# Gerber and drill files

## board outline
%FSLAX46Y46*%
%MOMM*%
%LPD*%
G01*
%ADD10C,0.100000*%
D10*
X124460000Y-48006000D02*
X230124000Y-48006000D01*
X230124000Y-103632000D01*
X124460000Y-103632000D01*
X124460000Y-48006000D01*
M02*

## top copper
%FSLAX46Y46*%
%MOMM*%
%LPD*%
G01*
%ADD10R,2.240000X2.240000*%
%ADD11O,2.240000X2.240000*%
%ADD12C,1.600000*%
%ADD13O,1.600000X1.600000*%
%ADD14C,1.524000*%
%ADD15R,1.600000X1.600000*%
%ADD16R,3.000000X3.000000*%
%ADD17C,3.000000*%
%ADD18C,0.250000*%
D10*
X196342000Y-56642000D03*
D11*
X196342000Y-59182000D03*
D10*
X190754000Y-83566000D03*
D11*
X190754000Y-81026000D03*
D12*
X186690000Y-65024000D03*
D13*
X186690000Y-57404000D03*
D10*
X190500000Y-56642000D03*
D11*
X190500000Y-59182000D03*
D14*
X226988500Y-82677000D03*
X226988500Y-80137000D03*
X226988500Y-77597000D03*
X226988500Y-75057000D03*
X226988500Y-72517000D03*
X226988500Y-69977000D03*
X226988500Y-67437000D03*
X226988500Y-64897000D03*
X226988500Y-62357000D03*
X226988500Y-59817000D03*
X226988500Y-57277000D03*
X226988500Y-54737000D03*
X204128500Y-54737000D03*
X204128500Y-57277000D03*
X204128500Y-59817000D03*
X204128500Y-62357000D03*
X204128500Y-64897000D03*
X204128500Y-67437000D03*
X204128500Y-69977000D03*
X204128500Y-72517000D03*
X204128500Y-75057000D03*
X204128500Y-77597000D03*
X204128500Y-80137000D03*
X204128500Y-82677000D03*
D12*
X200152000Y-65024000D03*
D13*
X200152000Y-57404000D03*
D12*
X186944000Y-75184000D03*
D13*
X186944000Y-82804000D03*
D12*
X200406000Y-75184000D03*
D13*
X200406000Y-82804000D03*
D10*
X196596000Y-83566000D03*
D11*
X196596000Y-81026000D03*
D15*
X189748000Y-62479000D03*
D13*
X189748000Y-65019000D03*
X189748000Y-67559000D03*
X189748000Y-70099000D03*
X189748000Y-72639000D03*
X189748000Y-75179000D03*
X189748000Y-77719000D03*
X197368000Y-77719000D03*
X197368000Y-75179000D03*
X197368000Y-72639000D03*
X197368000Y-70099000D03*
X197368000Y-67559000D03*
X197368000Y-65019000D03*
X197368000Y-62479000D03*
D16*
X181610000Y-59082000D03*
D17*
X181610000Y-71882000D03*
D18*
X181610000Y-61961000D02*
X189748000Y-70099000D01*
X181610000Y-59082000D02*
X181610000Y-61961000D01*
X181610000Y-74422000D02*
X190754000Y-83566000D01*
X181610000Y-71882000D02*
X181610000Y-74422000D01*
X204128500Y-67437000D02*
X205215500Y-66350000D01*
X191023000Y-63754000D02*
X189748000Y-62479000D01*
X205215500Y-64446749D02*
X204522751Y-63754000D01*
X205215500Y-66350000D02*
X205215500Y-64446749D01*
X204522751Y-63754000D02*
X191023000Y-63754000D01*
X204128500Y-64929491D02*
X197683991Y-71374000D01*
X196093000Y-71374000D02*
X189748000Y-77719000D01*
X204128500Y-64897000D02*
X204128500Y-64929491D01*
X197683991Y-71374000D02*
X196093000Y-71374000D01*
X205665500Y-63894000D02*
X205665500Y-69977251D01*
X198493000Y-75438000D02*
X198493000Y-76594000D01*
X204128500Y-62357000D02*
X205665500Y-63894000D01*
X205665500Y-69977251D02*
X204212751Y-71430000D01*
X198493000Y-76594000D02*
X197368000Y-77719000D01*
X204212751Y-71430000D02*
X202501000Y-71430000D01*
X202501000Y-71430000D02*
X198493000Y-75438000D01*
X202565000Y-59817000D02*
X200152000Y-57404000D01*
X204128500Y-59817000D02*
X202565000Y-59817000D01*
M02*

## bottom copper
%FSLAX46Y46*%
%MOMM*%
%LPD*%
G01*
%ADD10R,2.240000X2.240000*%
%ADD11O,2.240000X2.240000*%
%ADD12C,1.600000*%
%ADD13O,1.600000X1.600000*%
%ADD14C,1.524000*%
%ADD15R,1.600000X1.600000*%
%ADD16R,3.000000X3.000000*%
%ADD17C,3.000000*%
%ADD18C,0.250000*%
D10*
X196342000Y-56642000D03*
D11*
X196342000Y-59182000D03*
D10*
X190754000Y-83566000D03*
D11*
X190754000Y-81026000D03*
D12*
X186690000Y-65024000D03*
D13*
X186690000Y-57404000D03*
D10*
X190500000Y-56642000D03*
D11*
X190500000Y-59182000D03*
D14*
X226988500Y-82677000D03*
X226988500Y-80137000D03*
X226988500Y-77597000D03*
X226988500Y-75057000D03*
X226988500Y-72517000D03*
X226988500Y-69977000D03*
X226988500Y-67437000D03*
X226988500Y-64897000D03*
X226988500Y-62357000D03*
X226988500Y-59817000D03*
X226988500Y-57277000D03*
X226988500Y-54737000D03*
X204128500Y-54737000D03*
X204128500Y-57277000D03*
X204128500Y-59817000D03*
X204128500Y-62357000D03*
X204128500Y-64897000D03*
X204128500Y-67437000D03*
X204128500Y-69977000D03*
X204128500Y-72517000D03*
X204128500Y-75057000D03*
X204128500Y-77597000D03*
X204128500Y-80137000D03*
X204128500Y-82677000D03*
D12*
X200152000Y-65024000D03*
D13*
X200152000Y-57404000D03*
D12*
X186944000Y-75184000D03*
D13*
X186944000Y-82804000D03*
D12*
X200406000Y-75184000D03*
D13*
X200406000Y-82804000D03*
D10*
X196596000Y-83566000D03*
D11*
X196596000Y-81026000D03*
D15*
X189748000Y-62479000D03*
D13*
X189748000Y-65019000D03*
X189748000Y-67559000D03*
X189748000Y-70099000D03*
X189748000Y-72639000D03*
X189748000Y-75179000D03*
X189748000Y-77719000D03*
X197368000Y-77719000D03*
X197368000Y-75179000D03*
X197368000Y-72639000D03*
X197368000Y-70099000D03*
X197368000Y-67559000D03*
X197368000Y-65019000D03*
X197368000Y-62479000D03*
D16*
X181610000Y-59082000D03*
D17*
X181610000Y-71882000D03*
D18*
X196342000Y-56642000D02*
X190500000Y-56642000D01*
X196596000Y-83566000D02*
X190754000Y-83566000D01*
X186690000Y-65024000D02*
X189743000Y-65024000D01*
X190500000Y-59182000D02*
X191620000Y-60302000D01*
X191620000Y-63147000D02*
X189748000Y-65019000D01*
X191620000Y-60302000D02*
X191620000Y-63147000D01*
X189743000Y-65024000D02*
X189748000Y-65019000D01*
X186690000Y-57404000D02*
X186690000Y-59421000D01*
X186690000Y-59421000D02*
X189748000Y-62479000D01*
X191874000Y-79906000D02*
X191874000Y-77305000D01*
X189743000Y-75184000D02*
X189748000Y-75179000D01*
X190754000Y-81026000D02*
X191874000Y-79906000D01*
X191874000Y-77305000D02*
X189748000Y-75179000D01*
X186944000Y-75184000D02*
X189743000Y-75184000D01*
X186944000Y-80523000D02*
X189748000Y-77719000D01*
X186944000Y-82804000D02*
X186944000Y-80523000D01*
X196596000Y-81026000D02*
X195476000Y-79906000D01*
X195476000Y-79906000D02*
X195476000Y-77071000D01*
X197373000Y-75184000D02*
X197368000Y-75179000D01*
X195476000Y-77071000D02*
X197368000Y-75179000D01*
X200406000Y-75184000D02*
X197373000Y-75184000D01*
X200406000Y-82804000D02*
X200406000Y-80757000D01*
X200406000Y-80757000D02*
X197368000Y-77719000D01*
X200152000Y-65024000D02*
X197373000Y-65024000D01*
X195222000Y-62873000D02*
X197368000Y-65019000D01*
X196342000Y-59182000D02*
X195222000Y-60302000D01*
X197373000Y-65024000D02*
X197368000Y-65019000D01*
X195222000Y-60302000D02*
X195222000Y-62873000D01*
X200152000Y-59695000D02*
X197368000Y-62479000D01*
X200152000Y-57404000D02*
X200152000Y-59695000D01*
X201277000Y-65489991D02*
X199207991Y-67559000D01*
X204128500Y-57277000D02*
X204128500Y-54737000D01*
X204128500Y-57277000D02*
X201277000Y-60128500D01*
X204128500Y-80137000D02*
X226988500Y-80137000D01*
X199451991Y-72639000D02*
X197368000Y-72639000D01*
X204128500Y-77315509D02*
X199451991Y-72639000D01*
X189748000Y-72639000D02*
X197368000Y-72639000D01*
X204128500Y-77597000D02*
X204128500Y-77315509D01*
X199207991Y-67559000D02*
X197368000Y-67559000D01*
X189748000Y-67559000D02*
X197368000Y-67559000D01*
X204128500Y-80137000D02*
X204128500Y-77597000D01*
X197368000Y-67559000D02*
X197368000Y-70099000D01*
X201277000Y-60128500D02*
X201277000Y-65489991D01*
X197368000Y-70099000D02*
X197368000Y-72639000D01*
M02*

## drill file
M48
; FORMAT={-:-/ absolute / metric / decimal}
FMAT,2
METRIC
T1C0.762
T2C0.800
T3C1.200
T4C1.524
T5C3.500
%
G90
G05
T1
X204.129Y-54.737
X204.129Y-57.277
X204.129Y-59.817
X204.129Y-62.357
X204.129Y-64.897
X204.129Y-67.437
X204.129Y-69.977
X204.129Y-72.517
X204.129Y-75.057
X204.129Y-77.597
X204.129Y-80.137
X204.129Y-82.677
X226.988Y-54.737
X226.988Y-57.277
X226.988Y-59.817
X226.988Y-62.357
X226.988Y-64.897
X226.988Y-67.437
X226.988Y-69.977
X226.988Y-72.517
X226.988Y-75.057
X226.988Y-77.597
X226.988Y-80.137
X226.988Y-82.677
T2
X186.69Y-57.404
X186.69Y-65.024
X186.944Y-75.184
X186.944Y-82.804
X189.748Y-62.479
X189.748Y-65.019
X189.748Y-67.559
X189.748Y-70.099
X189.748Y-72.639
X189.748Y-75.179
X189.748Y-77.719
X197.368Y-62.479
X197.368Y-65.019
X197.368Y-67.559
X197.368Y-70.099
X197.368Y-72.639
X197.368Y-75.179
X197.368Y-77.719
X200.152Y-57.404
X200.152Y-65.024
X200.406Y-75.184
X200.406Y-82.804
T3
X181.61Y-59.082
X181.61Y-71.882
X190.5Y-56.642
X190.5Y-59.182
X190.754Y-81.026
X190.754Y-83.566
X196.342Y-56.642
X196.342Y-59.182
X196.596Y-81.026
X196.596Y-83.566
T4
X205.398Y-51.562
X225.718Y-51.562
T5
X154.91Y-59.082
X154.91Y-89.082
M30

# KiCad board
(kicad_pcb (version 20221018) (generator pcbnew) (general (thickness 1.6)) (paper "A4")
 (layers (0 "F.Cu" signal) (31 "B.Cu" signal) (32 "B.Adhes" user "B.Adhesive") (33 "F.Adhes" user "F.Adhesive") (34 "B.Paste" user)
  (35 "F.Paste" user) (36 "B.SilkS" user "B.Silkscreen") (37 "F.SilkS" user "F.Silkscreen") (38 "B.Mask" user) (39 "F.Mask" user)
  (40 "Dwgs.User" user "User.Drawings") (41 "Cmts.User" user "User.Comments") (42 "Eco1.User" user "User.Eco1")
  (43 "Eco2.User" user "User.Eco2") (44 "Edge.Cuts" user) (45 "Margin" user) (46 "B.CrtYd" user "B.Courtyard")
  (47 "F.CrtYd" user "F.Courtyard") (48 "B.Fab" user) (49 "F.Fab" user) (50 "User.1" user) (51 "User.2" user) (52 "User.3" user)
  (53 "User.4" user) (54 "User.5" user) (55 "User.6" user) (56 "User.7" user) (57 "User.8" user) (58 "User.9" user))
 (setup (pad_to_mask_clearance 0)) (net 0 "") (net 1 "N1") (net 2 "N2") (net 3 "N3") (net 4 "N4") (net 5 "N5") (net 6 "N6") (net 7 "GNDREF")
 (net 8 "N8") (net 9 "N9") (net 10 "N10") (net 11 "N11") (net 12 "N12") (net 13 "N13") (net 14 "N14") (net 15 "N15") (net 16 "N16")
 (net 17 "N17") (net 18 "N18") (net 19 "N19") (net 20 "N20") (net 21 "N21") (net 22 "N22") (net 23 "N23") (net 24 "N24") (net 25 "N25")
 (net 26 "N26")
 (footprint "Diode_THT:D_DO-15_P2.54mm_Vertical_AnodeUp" (layer "F.Cu") (at 196.342 56.642 -90)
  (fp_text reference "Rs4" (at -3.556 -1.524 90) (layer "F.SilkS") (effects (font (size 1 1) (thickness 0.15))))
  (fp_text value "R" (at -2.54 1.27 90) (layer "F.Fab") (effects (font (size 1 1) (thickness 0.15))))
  (pad "1" thru_hole rect (at 0 0 270) (size 2.24 2.24) (drill 1.2) (layers "*.Cu" "*.Mask") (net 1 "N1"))
  (pad "2" thru_hole oval (at 2.54 0 270) (size 2.24 2.24) (drill 1.2) (layers "*.Cu" "*.Mask") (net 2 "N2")))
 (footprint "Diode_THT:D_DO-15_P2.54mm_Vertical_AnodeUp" (layer "F.Cu") (at 190.754 83.566 90)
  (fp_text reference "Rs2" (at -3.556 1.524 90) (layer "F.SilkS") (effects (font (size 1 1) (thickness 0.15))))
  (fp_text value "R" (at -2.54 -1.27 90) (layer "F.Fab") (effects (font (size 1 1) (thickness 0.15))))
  (pad "1" thru_hole rect (at 0 0 90) (size 2.24 2.24) (drill 1.2) (layers "*.Cu" "*.Mask") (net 1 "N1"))
  (pad "2" thru_hole oval (at 2.54 0 90) (size 2.24 2.24) (drill 1.2) (layers "*.Cu" "*.Mask") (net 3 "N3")))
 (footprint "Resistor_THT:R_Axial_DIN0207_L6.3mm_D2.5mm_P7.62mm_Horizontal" (layer "F.Cu") (at 186.69 65.024 90)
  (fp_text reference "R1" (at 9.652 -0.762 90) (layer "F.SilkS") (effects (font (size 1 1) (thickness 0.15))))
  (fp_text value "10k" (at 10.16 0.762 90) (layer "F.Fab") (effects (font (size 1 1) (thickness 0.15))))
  (pad "1" thru_hole circle (at 0 0 90) (size 1.6 1.6) (drill 0.8) (layers "*.Cu" "*.Mask") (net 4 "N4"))
  (pad "2" thru_hole oval (at 7.62 0 90) (size 1.6 1.6) (drill 0.8) (layers "*.Cu" "*.Mask") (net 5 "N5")))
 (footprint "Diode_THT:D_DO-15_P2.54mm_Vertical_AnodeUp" (layer "F.Cu") (at 190.5 56.642 -90)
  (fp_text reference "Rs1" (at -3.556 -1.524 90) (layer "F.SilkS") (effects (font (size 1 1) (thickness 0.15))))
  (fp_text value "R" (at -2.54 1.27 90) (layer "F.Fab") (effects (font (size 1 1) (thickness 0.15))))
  (pad "1" thru_hole rect (at 0 0 270) (size 2.24 2.24) (drill 1.2) (layers "*.Cu" "*.Mask") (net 1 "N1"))
  (pad "2" thru_hole oval (at 2.54 0 270) (size 2.24 2.24) (drill 1.2) (layers "*.Cu" "*.Mask") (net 4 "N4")))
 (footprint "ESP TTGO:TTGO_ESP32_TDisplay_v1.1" (layer "F.Cu") (at 228.2585 99.187 90)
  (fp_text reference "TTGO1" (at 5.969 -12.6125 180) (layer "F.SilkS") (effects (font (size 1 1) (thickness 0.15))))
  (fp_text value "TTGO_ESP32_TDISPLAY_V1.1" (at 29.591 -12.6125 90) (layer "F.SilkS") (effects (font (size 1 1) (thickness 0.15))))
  (pad "" np_thru_hole circle (at 47.625 -22.86 90) (size 1.524 1.524) (drill 1.524) (layers "*.Cu" "*.Mask"))
  (pad "" np_thru_hole circle (at 47.625 -2.54 90) (size 1.524 1.524) (drill 1.524) (layers "*.Cu" "*.Mask"))
  (pad "1" thru_hole circle (at 16.51 -1.27 90) (size 1.524 1.524) (drill 0.762) (layers "*.Cu" "*.Mask") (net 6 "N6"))
  (pad "2" thru_hole circle (at 19.05 -1.27 90) (size 1.524 1.524) (drill 0.762) (layers "*.Cu" "*.Mask") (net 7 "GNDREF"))
  (pad "3" thru_hole circle (at 21.59 -1.27 90) (size 1.524 1.524) (drill 0.762) (layers "*.Cu" "*.Mask") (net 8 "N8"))
  (pad "4" thru_hole circle (at 24.13 -1.27 90) (size 1.524 1.524) (drill 0.762) (layers "*.Cu" "*.Mask") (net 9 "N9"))
  (pad "5" thru_hole circle (at 26.67 -1.27 90) (size 1.524 1.524) (drill 0.762) (layers "*.Cu" "*.Mask") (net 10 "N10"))
  (pad "6" thru_hole circle (at 29.21 -1.27 90) (size 1.524 1.524) (drill 0.762) (layers "*.Cu" "*.Mask") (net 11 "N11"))
  (pad "7" thru_hole circle (at 31.75 -1.27 90) (size 1.524 1.524) (drill 0.762) (layers "*.Cu" "*.Mask") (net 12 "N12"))
  (pad "8" thru_hole circle (at 34.29 -1.27 90) (size 1.524 1.524) (drill 0.762) (layers "*.Cu" "*.Mask") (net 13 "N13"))
  (pad "9" thru_hole circle (at 36.83 -1.27 90) (size 1.524 1.524) (drill 0.762) (layers "*.Cu" "*.Mask") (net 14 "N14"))
  (pad "10" thru_hole circle (at 39.37 -1.27 90) (size 1.524 1.524) (drill 0.762) (layers "*.Cu" "*.Mask") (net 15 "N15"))
  (pad "11" thru_hole circle (at 41.91 -1.27 90) (size 1.524 1.524) (drill 0.762) (layers "*.Cu" "*.Mask") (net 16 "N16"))
  (pad "12" thru_hole circle (at 44.45 -1.27 90) (size 1.524 1.524) (drill 0.762) (layers "*.Cu" "*.Mask") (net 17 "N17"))
  (pad "13" thru_hole circle (at 44.45 -24.13 90) (size 1.524 1.524) (drill 0.762) (layers "*.Cu" "*.Mask") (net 7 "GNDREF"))
  (pad "14" thru_hole circle (at 41.91 -24.13 90) (size 1.524 1.524) (drill 0.762) (layers "*.Cu" "*.Mask") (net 7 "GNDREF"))
  (pad "15" thru_hole circle (at 39.37 -24.13 90) (size 1.524 1.524) (drill 0.762) (layers "*.Cu" "*.Mask") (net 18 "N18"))
  (pad "16" thru_hole circle (at 36.83 -24.13 90) (size 1.524 1.524) (drill 0.762) (layers "*.Cu" "*.Mask") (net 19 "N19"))
  (pad "17" thru_hole circle (at 34.29 -24.13 90) (size 1.524 1.524) (drill 0.762) (layers "*.Cu" "*.Mask") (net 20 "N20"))
  (pad "18" thru_hole circle (at 31.75 -24.13 90) (size 1.524 1.524) (drill 0.762) (layers "*.Cu" "*.Mask") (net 5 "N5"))
  (pad "19" thru_hole circle (at 29.21 -24.13 90) (size 1.524 1.524) (drill 0.762) (layers "*.Cu" "*.Mask") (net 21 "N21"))
  (pad "20" thru_hole circle (at 26.67 -24.13 90) (size 1.524 1.524) (drill 0.762) (layers "*.Cu" "*.Mask") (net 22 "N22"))
  (pad "21" thru_hole circle (at 24.13 -24.13 90) (size 1.524 1.524) (drill 0.762) (layers "*.Cu" "*.Mask") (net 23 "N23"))
  (pad "22" thru_hole circle (at 21.59 -24.13 90) (size 1.524 1.524) (drill 0.762) (layers "*.Cu" "*.Mask") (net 7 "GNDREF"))
  (pad "23" thru_hole circle (at 19.05 -24.13 90) (size 1.524 1.524) (drill 0.762) (layers "*.Cu" "*.Mask") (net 7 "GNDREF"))
  (pad "24" thru_hole circle (at 16.51 -24.13 90) (size 1.524 1.524) (drill 0.762) (layers "*.Cu" "*.Mask") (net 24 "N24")))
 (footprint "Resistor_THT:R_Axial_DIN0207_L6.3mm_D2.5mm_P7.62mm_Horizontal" (layer "F.Cu") (at 200.152 65.024 90)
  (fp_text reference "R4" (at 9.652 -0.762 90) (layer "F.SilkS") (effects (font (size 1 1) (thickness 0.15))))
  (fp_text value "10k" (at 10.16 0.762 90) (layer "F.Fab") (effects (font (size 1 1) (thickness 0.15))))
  (pad "1" thru_hole circle (at 0 0 90) (size 1.6 1.6) (drill 0.8) (layers "*.Cu" "*.Mask") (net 2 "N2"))
  (pad "2" thru_hole oval (at 7.62 0 90) (size 1.6 1.6) (drill 0.8) (layers "*.Cu" "*.Mask") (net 18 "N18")))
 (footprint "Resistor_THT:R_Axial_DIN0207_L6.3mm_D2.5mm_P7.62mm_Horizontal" (layer "F.Cu") (at 186.944 75.184 -90)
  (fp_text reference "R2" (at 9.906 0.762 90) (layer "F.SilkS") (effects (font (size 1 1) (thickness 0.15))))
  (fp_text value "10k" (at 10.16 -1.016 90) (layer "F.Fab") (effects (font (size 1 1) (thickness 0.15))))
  (pad "1" thru_hole circle (at 0 0 270) (size 1.6 1.6) (drill 0.8) (layers "*.Cu" "*.Mask") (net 3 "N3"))
  (pad "2" thru_hole oval (at 7.62 0 270) (size 1.6 1.6) (drill 0.8) (layers "*.Cu" "*.Mask") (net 20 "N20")))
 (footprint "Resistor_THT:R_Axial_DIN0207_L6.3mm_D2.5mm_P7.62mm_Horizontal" (layer "F.Cu") (at 200.406 75.184 -90)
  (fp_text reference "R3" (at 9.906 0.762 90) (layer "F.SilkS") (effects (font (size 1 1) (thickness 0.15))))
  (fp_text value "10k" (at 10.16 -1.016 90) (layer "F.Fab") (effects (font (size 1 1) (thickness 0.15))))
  (pad "1" thru_hole circle (at 0 0 270) (size 1.6 1.6) (drill 0.8) (layers "*.Cu" "*.Mask") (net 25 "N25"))
  (pad "2" thru_hole oval (at 7.62 0 270) (size 1.6 1.6) (drill 0.8) (layers "*.Cu" "*.Mask") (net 19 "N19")))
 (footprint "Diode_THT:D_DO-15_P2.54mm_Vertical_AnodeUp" (layer "F.Cu") (at 196.596 83.566 90)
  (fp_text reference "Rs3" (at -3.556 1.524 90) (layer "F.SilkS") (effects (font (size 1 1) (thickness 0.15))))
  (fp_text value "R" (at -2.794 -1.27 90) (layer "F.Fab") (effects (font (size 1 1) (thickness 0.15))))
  (pad "1" thru_hole rect (at 0 0 90) (size 2.24 2.24) (drill 1.2) (layers "*.Cu" "*.Mask") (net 1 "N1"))
  (pad "2" thru_hole oval (at 2.54 0 90) (size 2.24 2.24) (drill 1.2) (layers "*.Cu" "*.Mask") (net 25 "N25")))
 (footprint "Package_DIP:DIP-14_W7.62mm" (layer "F.Cu") (at 189.748 62.479)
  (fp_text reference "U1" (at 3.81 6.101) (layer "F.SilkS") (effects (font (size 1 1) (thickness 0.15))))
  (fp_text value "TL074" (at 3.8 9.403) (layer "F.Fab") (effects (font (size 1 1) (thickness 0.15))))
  (pad "1" thru_hole rect (at 0 0) (size 1.6 1.6) (drill 0.8) (layers "*.Cu" "*.Mask") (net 5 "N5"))
  (pad "2" thru_hole oval (at 0 2.54) (size 1.6 1.6) (drill 0.8) (layers "*.Cu" "*.Mask") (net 4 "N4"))
  (pad "3" thru_hole oval (at 0 5.08) (size 1.6 1.6) (drill 0.8) (layers "*.Cu" "*.Mask") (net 7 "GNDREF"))
  (pad "4" thru_hole oval (at 0 7.62) (size 1.6 1.6) (drill 0.8) (layers "*.Cu" "*.Mask") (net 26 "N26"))
  (pad "5" thru_hole oval (at 0 10.16) (size 1.6 1.6) (drill 0.8) (layers "*.Cu" "*.Mask") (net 7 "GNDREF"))
  (pad "6" thru_hole oval (at 0 12.7) (size 1.6 1.6) (drill 0.8) (layers "*.Cu" "*.Mask") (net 3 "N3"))
  (pad "7" thru_hole oval (at 0 15.24) (size 1.6 1.6) (drill 0.8) (layers "*.Cu" "*.Mask") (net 20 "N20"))
  (pad "8" thru_hole oval (at 7.62 15.24) (size 1.6 1.6) (drill 0.8) (layers "*.Cu" "*.Mask") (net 19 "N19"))
  (pad "9" thru_hole oval (at 7.62 12.7) (size 1.6 1.6) (drill 0.8) (layers "*.Cu" "*.Mask") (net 25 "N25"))
  (pad "10" thru_hole oval (at 7.62 10.16) (size 1.6 1.6) (drill 0.8) (layers "*.Cu" "*.Mask") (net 7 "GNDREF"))
  (pad "11" thru_hole oval (at 7.62 7.62) (size 1.6 1.6) (drill 0.8) (layers "*.Cu" "*.Mask") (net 7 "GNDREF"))
  (pad "12" thru_hole oval (at 7.62 5.08) (size 1.6 1.6) (drill 0.8) (layers "*.Cu" "*.Mask") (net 7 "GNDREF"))
  (pad "13" thru_hole oval (at 7.62 2.54) (size 1.6 1.6) (drill 0.8) (layers "*.Cu" "*.Mask") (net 2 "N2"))
  (pad "14" thru_hole oval (at 7.62 0) (size 1.6 1.6) (drill 0.8) (layers "*.Cu" "*.Mask") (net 18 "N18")))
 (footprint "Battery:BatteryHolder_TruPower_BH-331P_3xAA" (layer "B.Cu") (at 181.61 59.082 180)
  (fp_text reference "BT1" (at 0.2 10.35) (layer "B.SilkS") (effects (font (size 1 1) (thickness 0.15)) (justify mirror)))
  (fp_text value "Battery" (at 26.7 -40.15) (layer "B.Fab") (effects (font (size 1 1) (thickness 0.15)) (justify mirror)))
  (pad "" np_thru_hole circle (at 26.7 -30 180) (size 3.5 3.5) (drill 3.5) (layers "*.Cu" "*.Mask"))
  (pad "" np_thru_hole circle (at 26.7 0 180) (size 3.5 3.5) (drill 3.5) (layers "*.Cu" "*.Mask"))
  (pad "1" thru_hole rect (at 0 0 180) (size 3 3) (drill 1.2) (layers "*.Cu" "*.Mask") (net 26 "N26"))
  (pad "2" thru_hole circle (at 0 -12.8 180) (size 3 3) (drill 1.2) (layers "*.Cu" "*.Mask") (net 1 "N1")))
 (gr_rect (start 124.46 48.006) (end 230.124 103.632) (stroke (width 0.1) (type default)) (fill none) (layer "Edge.Cuts"))
 (segment (start 181.61 61.961) (end 189.748 70.099) (width 0.25) (layer "F.Cu") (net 26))
 (segment (start 181.61 59.082) (end 181.61 61.961) (width 0.25) (layer "F.Cu") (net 26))
 (segment (start 181.61 74.422) (end 190.754 83.566) (width 0.25) (layer "F.Cu") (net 1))
 (segment (start 181.61 71.882) (end 181.61 74.422) (width 0.25) (layer "F.Cu") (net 1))
 (segment (start 196.342 56.642) (end 190.5 56.642) (width 0.25) (layer "B.Cu") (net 1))
 (segment (start 196.596 83.566) (end 190.754 83.566) (width 0.25) (layer "B.Cu") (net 1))
 (segment (start 186.69 65.024) (end 189.743 65.024) (width 0.25) (layer "B.Cu") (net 4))
 (segment (start 190.5 59.182) (end 191.62 60.302) (width 0.25) (layer "B.Cu") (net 4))
 (segment (start 191.62 63.147) (end 189.748 65.019) (width 0.25) (layer "B.Cu") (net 4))
 (segment (start 191.62 60.302) (end 191.62 63.147) (width 0.25) (layer "B.Cu") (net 4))
 (segment (start 189.743 65.024) (end 189.748 65.019) (width 0.25) (layer "B.Cu") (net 4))
 (segment (start 204.1285 67.437) (end 205.2155 66.35) (width 0.25) (layer "F.Cu") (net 5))
 (segment (start 191.023 63.754) (end 189.748 62.479) (width 0.25) (layer "F.Cu") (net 5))
 (segment (start 205.2155 64.446749) (end 204.522751 63.754) (width 0.25) (layer "F.Cu") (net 5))
 (segment (start 205.2155 66.35) (end 205.2155 64.446749) (width 0.25) (layer "F.Cu") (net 5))
 (segment (start 204.522751 63.754) (end 191.023 63.754) (width 0.25) (layer "F.Cu") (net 5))
 (segment (start 186.69 57.404) (end 186.69 59.421) (width 0.25) (layer "B.Cu") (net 5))
 (segment (start 186.69 59.421) (end 189.748 62.479) (width 0.25) (layer "B.Cu") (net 5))
 (segment (start 191.874 79.906) (end 191.874 77.305) (width 0.25) (layer "B.Cu") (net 3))
 (segment (start 189.743 75.184) (end 189.748 75.179) (width 0.25) (layer "B.Cu") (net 3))
 (segment (start 190.754 81.026) (end 191.874 79.906) (width 0.25) (layer "B.Cu") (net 3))
 (segment (start 191.874 77.305) (end 189.748 75.179) (width 0.25) (layer "B.Cu") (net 3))
 (segment (start 186.944 75.184) (end 189.743 75.184) (width 0.25) (layer "B.Cu") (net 3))
 (segment (start 204.1285 64.929491) (end 197.683991 71.374) (width 0.25) (layer "F.Cu") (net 20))
 (segment (start 196.093 71.374) (end 189.748 77.719) (width 0.25) (layer "F.Cu") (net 20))
 (segment (start 204.1285 64.897) (end 204.1285 64.929491) (width 0.25) (layer "F.Cu") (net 20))
 (segment (start 197.683991 71.374) (end 196.093 71.374) (width 0.25) (layer "F.Cu") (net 20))
 (segment (start 186.944 80.523) (end 189.748 77.719) (width 0.25) (layer "B.Cu") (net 20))
 (segment (start 186.944 82.804) (end 186.944 80.523) (width 0.25) (layer "B.Cu") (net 20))
 (segment (start 196.596 81.026) (end 195.476 79.906) (width 0.25) (layer "B.Cu") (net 25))
 (segment (start 195.476 79.906) (end 195.476 77.071) (width 0.25) (layer "B.Cu") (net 25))
 (segment (start 197.373 75.184) (end 197.368 75.179) (width 0.25) (layer "B.Cu") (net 25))
 (segment (start 195.476 77.071) (end 197.368 75.179) (width 0.25) (layer "B.Cu") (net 25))
 (segment (start 200.406 75.184) (end 197.373 75.184) (width 0.25) (layer "B.Cu") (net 25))
 (segment (start 205.6655 63.894) (end 205.6655 69.977251) (width 0.25) (layer "F.Cu") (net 19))
 (segment (start 198.493 75.438) (end 198.493 76.594) (width 0.25) (layer "F.Cu") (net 19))
 (segment (start 204.1285 62.357) (end 205.6655 63.894) (width 0.25) (layer "F.Cu") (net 19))
 (segment (start 205.6655 69.977251) (end 204.212751 71.43) (width 0.25) (layer "F.Cu") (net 19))
 (segment (start 198.493 76.594) (end 197.368 77.719) (width 0.25) (layer "F.Cu") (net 19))
 (segment (start 204.212751 71.43) (end 202.501 71.43) (width 0.25) (layer "F.Cu") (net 19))
 (segment (start 202.501 71.43) (end 198.493 75.438) (width 0.25) (layer "F.Cu") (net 19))
 (segment (start 200.406 82.804) (end 200.406 80.757) (width 0.25) (layer "B.Cu") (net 19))
 (segment (start 200.406 80.757) (end 197.368 77.719) (width 0.25) (layer "B.Cu") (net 19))
 (segment (start 200.152 65.024) (end 197.373 65.024) (width 0.25) (layer "B.Cu") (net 2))
 (segment (start 195.222 62.873) (end 197.368 65.019) (width 0.25) (layer "B.Cu") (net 2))
 (segment (start 196.342 59.182) (end 195.222 60.302) (width 0.25) (layer "B.Cu") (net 2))
 (segment (start 197.373 65.024) (end 197.368 65.019) (width 0.25) (layer "B.Cu") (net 2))
 (segment (start 195.222 60.302) (end 195.222 62.873) (width 0.25) (layer "B.Cu") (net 2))
 (segment (start 202.565 59.817) (end 200.152 57.404) (width 0.25) (layer "F.Cu") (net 18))
 (segment (start 204.1285 59.817) (end 202.565 59.817) (width 0.25) (layer "F.Cu") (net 18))
 (segment (start 200.152 59.695) (end 197.368 62.479) (width 0.25) (layer "B.Cu") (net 18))
 (segment (start 200.152 57.404) (end 200.152 59.695) (width 0.25) (layer "B.Cu") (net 18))
 (segment (start 201.277 65.489991) (end 199.207991 67.559) (width 0.25) (layer "B.Cu") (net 7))
 (segment (start 204.1285 57.277) (end 204.1285 54.737) (width 0.25) (layer "B.Cu") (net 7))
 (segment (start 204.1285 57.277) (end 201.277 60.1285) (width 0.25) (layer "B.Cu") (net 7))
 (segment (start 204.1285 80.137) (end 226.9885 80.137) (width 0.25) (layer "B.Cu") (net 7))
 (segment (start 199.451991 72.639) (end 197.368 72.639) (width 0.25) (layer "B.Cu") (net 7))
 (segment (start 204.1285 77.315509) (end 199.451991 72.639) (width 0.25) (layer "B.Cu") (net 7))
 (segment (start 189.748 72.639) (end 197.368 72.639) (width 0.25) (layer "B.Cu") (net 7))
 (segment (start 204.1285 77.597) (end 204.1285 77.315509) (width 0.25) (layer "B.Cu") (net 7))
 (segment (start 199.207991 67.559) (end 197.368 67.559) (width 0.25) (layer "B.Cu") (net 7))
 (segment (start 189.748 67.559) (end 197.368 67.559) (width 0.25) (layer "B.Cu") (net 7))
 (segment (start 204.1285 80.137) (end 204.1285 77.597) (width 0.25) (layer "B.Cu") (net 7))
 (segment (start 197.368 67.559) (end 197.368 70.099) (width 0.25) (layer "B.Cu") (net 7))
 (segment (start 201.277 60.1285) (end 201.277 65.489991) (width 0.25) (layer "B.Cu") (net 7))
 (segment (start 197.368 70.099) (end 197.368 72.639) (width 0.25) (layer "B.Cu") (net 7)))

